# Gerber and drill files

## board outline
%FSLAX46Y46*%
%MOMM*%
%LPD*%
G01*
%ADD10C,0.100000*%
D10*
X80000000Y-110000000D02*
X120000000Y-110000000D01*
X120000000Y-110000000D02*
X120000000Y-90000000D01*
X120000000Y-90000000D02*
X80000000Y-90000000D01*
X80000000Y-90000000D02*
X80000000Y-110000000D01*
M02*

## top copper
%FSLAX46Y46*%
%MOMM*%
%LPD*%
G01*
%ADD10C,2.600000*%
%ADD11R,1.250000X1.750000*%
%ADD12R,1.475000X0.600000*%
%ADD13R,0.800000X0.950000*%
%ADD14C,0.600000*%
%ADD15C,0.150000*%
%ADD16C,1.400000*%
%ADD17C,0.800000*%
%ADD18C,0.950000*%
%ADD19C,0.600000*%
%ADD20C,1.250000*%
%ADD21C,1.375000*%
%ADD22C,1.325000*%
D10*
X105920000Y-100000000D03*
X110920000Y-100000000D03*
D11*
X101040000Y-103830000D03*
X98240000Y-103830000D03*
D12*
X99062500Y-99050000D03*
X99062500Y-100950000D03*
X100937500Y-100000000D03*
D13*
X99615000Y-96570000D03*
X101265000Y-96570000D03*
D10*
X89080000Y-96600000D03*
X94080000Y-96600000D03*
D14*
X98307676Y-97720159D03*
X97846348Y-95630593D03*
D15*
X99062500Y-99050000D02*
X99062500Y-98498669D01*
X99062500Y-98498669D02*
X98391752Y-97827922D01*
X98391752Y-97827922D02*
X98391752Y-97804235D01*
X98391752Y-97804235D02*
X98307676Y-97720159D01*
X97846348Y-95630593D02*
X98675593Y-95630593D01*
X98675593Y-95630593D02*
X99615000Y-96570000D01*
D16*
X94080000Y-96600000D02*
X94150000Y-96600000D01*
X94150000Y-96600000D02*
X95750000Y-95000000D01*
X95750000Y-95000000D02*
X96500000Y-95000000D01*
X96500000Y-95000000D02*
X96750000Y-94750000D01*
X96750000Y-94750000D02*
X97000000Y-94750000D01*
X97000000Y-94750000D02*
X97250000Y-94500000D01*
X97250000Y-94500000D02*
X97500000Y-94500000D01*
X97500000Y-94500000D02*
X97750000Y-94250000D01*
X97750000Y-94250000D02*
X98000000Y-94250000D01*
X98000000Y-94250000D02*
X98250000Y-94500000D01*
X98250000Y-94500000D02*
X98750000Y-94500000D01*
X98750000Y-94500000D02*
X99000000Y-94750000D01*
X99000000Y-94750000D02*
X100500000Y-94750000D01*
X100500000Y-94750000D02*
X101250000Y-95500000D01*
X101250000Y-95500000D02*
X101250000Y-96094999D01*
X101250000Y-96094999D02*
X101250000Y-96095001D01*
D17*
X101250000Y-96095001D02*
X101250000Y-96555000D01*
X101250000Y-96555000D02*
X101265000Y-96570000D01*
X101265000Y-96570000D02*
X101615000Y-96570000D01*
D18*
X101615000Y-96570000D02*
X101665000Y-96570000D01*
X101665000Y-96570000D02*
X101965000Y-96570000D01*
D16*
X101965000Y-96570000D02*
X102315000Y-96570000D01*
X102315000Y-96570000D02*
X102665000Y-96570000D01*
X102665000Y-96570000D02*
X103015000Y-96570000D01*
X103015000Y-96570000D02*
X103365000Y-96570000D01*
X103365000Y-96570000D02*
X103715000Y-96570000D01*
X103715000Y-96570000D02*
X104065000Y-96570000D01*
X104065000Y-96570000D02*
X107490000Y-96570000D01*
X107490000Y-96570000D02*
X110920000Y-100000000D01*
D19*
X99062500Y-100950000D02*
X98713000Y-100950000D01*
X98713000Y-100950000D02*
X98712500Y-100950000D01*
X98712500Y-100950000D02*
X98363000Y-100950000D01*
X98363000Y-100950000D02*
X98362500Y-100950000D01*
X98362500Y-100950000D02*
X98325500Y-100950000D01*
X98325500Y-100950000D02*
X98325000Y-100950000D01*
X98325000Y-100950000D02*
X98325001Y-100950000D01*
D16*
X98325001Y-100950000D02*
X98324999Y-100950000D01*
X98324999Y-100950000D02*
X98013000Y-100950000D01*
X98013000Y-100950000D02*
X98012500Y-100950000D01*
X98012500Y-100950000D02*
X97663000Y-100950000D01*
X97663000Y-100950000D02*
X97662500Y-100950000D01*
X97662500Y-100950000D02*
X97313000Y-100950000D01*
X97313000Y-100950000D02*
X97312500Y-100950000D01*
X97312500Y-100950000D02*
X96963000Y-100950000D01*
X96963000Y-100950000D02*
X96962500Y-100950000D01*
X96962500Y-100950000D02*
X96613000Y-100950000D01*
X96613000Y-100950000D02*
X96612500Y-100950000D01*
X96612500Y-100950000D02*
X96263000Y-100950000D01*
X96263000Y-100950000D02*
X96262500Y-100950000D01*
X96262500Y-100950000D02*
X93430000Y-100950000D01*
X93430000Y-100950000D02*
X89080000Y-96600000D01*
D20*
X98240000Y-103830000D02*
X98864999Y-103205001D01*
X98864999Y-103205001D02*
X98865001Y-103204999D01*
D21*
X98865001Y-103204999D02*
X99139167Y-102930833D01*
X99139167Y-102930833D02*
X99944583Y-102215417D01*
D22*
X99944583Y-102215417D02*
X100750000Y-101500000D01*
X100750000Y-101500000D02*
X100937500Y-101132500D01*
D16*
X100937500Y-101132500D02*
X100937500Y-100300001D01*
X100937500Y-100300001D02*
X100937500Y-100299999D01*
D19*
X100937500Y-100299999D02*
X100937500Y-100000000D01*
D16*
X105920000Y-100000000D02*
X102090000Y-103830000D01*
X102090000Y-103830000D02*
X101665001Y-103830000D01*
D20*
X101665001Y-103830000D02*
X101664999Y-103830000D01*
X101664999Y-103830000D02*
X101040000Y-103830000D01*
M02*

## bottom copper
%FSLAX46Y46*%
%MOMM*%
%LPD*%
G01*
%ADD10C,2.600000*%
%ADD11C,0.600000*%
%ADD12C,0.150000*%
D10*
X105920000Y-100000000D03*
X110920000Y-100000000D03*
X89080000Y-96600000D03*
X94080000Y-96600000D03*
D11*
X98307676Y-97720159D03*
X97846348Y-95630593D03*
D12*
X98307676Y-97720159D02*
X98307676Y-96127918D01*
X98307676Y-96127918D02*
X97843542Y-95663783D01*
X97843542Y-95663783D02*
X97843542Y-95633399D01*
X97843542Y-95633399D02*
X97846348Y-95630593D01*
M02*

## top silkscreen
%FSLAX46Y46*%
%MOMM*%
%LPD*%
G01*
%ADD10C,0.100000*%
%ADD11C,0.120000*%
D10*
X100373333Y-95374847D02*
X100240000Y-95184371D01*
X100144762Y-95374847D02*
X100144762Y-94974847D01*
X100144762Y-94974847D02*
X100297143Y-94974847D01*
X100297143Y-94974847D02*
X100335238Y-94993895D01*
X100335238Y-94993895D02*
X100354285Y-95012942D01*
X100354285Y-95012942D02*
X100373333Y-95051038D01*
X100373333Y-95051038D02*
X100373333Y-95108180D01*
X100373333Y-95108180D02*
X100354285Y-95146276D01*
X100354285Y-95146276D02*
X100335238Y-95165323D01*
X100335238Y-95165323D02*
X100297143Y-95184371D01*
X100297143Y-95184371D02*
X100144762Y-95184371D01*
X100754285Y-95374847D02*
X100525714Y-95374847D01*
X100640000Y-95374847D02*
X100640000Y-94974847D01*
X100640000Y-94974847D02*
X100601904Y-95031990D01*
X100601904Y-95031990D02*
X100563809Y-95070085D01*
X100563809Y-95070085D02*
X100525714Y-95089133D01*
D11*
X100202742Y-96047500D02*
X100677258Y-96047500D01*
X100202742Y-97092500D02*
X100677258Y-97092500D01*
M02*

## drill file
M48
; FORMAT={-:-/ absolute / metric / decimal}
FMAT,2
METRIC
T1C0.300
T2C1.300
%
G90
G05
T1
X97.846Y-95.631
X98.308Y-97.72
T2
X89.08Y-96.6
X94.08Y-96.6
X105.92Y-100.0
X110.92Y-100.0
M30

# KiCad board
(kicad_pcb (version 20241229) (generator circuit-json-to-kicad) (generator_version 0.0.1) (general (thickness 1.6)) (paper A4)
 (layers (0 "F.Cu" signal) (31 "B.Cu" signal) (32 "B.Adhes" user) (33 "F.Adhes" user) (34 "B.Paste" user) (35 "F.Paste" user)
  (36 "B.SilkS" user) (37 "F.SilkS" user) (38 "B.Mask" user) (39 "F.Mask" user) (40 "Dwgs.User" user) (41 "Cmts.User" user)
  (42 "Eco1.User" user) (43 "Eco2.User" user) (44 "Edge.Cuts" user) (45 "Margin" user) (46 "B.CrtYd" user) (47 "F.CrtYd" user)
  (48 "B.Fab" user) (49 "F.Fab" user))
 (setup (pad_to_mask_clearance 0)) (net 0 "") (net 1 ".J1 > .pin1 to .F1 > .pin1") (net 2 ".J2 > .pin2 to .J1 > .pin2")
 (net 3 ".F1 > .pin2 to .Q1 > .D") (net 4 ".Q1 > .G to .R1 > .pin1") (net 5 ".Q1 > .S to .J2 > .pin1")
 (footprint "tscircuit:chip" (layer F.Cu) (at 105.92 100 0)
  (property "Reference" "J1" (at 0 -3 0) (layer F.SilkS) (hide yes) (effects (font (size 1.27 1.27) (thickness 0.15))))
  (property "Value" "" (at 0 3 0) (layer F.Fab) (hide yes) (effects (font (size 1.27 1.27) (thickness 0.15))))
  (pad "1" thru_hole circle (at 0 0 0) (size 2.6 2.6) (drill 1.3) (layers *.Cu *.Mask) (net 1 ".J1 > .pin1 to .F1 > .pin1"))
  (pad "2" thru_hole circle (at 5 0 0) (size 2.6 2.6) (drill 1.3) (layers *.Cu *.Mask) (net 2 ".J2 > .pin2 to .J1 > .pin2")))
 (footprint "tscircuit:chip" (layer F.Cu) (at 99.64 103.83 180)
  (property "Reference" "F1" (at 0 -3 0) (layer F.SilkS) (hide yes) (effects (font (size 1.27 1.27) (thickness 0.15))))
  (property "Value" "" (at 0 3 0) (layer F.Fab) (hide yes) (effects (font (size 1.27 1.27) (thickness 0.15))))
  (pad "1" smd rect (at -1.4 0 0) (size 1.25 1.75) (layers F.Cu F.Mask) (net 1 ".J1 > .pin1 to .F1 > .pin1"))
  (pad "2" smd rect (at 1.4 0 0) (size 1.25 1.75) (layers F.Cu F.Mask) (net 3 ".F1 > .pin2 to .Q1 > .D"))
  (pad "" smd rect (at -1.4 0 0) (size 0.875 1.2249999999999999) (layers F.Paste))
  (pad "" smd rect (at 1.4 0 0) (size 0.875 1.2249999999999999) (layers F.Paste)))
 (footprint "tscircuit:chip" (layer F.Cu) (at 100 100 0)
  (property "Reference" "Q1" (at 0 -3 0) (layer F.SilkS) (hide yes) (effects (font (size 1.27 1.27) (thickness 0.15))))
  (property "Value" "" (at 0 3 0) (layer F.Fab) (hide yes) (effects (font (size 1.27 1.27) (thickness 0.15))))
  (pad "1" smd rect (at -0.9375 -0.95 0) (size 1.475 0.6) (layers F.Cu F.Mask) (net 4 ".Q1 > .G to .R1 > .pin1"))
  (pad "2" smd rect (at -0.9375 0.95 0) (size 1.475 0.6) (layers F.Cu F.Mask) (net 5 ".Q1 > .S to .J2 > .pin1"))
  (pad "3" smd rect (at 0.9375 0 0) (size 1.475 0.6) (layers F.Cu F.Mask) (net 3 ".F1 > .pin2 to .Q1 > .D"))
  (pad "" smd rect (at -0.9375 -0.95 0) (size 1.0325 0.42) (layers F.Paste))
  (pad "" smd rect (at -0.9375 0.95 0) (size 1.0325 0.42) (layers F.Paste))
  (pad "" smd rect (at 0.9375 0 0) (size 1.0325 0.42) (layers F.Paste)))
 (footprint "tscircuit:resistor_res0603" (layer F.Cu) (at 100.44 96.57 0)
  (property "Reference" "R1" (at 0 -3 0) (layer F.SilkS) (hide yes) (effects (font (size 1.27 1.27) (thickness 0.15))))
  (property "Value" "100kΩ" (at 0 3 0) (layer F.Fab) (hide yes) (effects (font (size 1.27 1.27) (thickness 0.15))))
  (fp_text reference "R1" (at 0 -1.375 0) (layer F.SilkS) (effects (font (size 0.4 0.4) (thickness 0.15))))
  (fp_line (start -0.237258 -0.5225) (end 0.23725799999999997 -0.5225) (stroke (width 0.12) (type default)) (layer F.SilkS))
  (fp_line (start -0.237258 0.5225) (end 0.23725799999999997 0.5225) (stroke (width 0.12) (type default)) (layer F.SilkS))
  (pad "1" smd rect (at -0.825 0 0) (size 0.8 0.95) (layers F.Cu F.Mask) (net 4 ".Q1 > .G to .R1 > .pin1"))
  (pad "2" smd rect (at 0.825 0 0) (size 0.8 0.95) (layers F.Cu F.Mask) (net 2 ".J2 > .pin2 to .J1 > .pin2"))
  (pad "" smd rect (at -0.825 0 0) (size 0.5599999999999999 0.6649999999999999) (layers F.Paste))
  (pad "" smd rect (at 0.825 0 0) (size 0.5599999999999999 0.6649999999999999) (layers F.Paste)))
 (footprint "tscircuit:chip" (layer F.Cu) (at 89.08 96.6 0)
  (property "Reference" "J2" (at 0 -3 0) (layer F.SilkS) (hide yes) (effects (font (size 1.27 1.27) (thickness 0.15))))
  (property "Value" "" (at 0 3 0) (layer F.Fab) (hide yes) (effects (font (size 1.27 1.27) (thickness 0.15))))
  (pad "1" thru_hole circle (at 0 0 0) (size 2.6 2.6) (drill 1.3) (layers *.Cu *.Mask) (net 5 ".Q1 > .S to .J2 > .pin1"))
  (pad "2" thru_hole circle (at 5 0 0) (size 2.6 2.6) (drill 1.3) (layers *.Cu *.Mask) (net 2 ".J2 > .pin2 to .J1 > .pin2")))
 (segment (start 99.0625 99.05) (end 99.0625 98.49866917639389) (width 0.15) (layer F.Cu) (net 4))
 (segment (start 99.0625 98.49866917639389) (end 98.39175243083571 97.82792160722961) (width 0.15) (layer F.Cu) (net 4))
 (segment (start 98.39175243083571 97.82792160722961) (end 98.39175243083571 97.80423524011546) (width 0.15) (layer F.Cu) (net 4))
 (segment (start 98.39175243083571 97.80423524011546) (end 98.30767637246909 97.72015918174884) (width 0.15) (layer F.Cu) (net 4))
 (segment (start 98.30767637246909 97.72015918174884) (end 98.30767637246909 96.12791807272515) (width 0.15) (layer B.Cu) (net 4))
 (segment (start 98.30767637246909 96.12791807272515) (end 97.84354177922641 95.66378347948246) (width 0.15) (layer B.Cu) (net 4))
 (segment (start 97.84354177922641 95.66378347948246) (end 97.84354177922641 95.63339917294248) (width 0.15) (layer B.Cu) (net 4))
 (segment (start 97.84354177922641 95.63339917294248) (end 97.8463483227921 95.63059262937678) (width 0.15) (layer B.Cu) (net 4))
 (segment (start 97.8463483227921 95.63059262937678) (end 98.67559262937678 95.63059262937678) (width 0.15) (layer F.Cu) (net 4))
 (segment (start 98.67559262937678 95.63059262937678) (end 99.615 96.57) (width 0.15) (layer F.Cu) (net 4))
 (segment (start 94.08 96.6) (end 94.15 96.6) (width 1.4) (layer F.Cu) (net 2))
 (segment (start 94.15 96.6) (end 95.75 95) (width 1.4) (layer F.Cu) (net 2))
 (segment (start 95.75 95) (end 96.5 95) (width 1.4) (layer F.Cu) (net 2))
 (segment (start 96.5 95) (end 96.75 94.75) (width 1.4) (layer F.Cu) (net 2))
 (segment (start 96.75 94.75) (end 97 94.75) (width 1.4) (layer F.Cu) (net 2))
 (segment (start 97 94.75) (end 97.25 94.5) (width 1.4) (layer F.Cu) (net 2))
 (segment (start 97.25 94.5) (end 97.5 94.5) (width 1.4) (layer F.Cu) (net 2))
 (segment (start 97.5 94.5) (end 97.75 94.25) (width 1.4) (layer F.Cu) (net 2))
 (segment (start 97.75 94.25) (end 98 94.25) (width 1.4) (layer F.Cu) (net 2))
 (segment (start 98 94.25) (end 98.25 94.5) (width 1.4) (layer F.Cu) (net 2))
 (segment (start 98.25 94.5) (end 98.75 94.5) (width 1.4) (layer F.Cu) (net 2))
 (segment (start 98.75 94.5) (end 99 94.75) (width 1.4) (layer F.Cu) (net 2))
 (segment (start 99 94.75) (end 100.5 94.75) (width 1.4) (layer F.Cu) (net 2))
 (segment (start 100.5 94.75) (end 101.25 95.5) (width 1.4) (layer F.Cu) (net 2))
 (segment (start 101.25 95.5) (end 101.25 96.094999) (width 1.4) (layer F.Cu) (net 2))
 (segment (start 101.25 96.094999) (end 101.25 96.095001) (width 1.4) (layer F.Cu) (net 2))
 (segment (start 101.25 96.095001) (end 101.25 96.555) (width 0.8) (layer F.Cu) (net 2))
 (segment (start 101.25 96.555) (end 101.265 96.57) (width 0.8) (layer F.Cu) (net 2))
 (segment (start 101.265 96.57) (end 101.615 96.57) (width 0.8) (layer F.Cu) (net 2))
 (segment (start 101.615 96.57) (end 101.665 96.57) (width 0.95) (layer F.Cu) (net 2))
 (segment (start 101.665 96.57) (end 101.965 96.57) (width 0.95) (layer F.Cu) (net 2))
 (segment (start 101.965 96.57) (end 102.315 96.57) (width 1.4) (layer F.Cu) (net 2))
 (segment (start 102.315 96.57) (end 102.665 96.57) (width 1.4) (layer F.Cu) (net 2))
 (segment (start 102.665 96.57) (end 103.015 96.57) (width 1.4) (layer F.Cu) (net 2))
 (segment (start 103.015 96.57) (end 103.365 96.57) (width 1.4) (layer F.Cu) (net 2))
 (segment (start 103.365 96.57) (end 103.715 96.57) (width 1.4) (layer F.Cu) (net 2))
 (segment (start 103.715 96.57) (end 104.065 96.57) (width 1.4) (layer F.Cu) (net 2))
 (segment (start 104.065 96.57) (end 107.49 96.57) (width 1.4) (layer F.Cu) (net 2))
 (segment (start 107.49 96.57) (end 110.92 100) (width 1.4) (layer F.Cu) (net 2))
 (segment (start 99.0625 100.95) (end 98.713 100.95) (width 0.6) (layer F.Cu) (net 5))
 (segment (start 98.713 100.95) (end 98.7125 100.95) (width 0.6) (layer F.Cu) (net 5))
 (segment (start 98.7125 100.95) (end 98.363 100.95) (width 0.6) (layer F.Cu) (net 5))
 (segment (start 98.363 100.95) (end 98.3625 100.95) (width 0.6) (layer F.Cu) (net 5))
 (segment (start 98.3625 100.95) (end 98.3255 100.95) (width 0.6) (layer F.Cu) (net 5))
 (segment (start 98.3255 100.95) (end 98.325 100.95) (width 0.6) (layer F.Cu) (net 5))
 (segment (start 98.325 100.95) (end 98.325001 100.95) (width 0.6) (layer F.Cu) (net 5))
 (segment (start 98.325001 100.95) (end 98.324999 100.95) (width 1.4) (layer F.Cu) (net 5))
 (segment (start 98.324999 100.95) (end 98.013 100.95) (width 1.4) (layer F.Cu) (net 5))
 (segment (start 98.013 100.95) (end 98.0125 100.95) (width 1.4) (layer F.Cu) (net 5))
 (segment (start 98.0125 100.95) (end 97.663 100.95) (width 1.4) (layer F.Cu) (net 5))
 (segment (start 97.663 100.95) (end 97.6625 100.95) (width 1.4) (layer F.Cu) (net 5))
 (segment (start 97.6625 100.95) (end 97.313 100.95) (width 1.4) (layer F.Cu) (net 5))
 (segment (start 97.313 100.95) (end 97.3125 100.95) (width 1.4) (layer F.Cu) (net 5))
 (segment (start 97.3125 100.95) (end 96.963 100.95) (width 1.4) (layer F.Cu) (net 5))
 (segment (start 96.963 100.95) (end 96.9625 100.95) (width 1.4) (layer F.Cu) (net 5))
 (segment (start 96.9625 100.95) (end 96.613 100.95) (width 1.4) (layer F.Cu) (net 5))
 (segment (start 96.613 100.95) (end 96.6125 100.95) (width 1.4) (layer F.Cu) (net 5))
 (segment (start 96.6125 100.95) (end 96.263 100.95) (width 1.4) (layer F.Cu) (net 5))
 (segment (start 96.263 100.95) (end 96.2625 100.95) (width 1.4) (layer F.Cu) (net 5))
 (segment (start 96.2625 100.95) (end 93.42999999999999 100.95) (width 1.4) (layer F.Cu) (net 5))
 (segment (start 93.42999999999999 100.95) (end 89.08 96.6) (width 1.4) (layer F.Cu) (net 5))
 (segment (start 98.24 103.83) (end 98.86499929289322 103.20500070710678) (width 1.25) (layer F.Cu) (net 3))
 (segment (start 98.86499929289322 103.20500070710678) (end 98.86500070710679 103.20499929289322) (width 1.25) (layer F.Cu) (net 3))
 (segment (start 98.86500070710679 103.20499929289322) (end 99.13916666666667 102.93083333333334) (width 1.375) (layer F.Cu) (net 3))
 (segment (start 99.13916666666667 102.93083333333334) (end 99.94458333333333 102.21541666666667) (width 1.375) (layer F.Cu) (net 3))
 (segment (start 99.94458333333333 102.21541666666667) (end 100.75 101.5) (width 1.3250000000000002) (layer F.Cu) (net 3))
 (segment (start 100.75 101.5) (end 100.9375 101.1325) (width 1.3250000000000002) (layer F.Cu) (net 3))
 (segment (start 100.9375 101.1325) (end 100.9375 100.300001) (width 1.4) (layer F.Cu) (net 3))
 (segment (start 100.9375 100.300001) (end 100.9375 100.299999) (width 1.4) (layer F.Cu) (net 3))
 (segment (start 100.9375 100.299999) (end 100.9375 100) (width 0.6) (layer F.Cu) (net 3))
 (segment (start 105.92 100) (end 102.09 103.83) (width 1.4) (layer F.Cu) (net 1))
 (segment (start 102.09 103.83) (end 101.665001 103.83) (width 1.4) (layer F.Cu) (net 1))
 (segment (start 101.665001 103.83) (end 101.664999 103.83) (width 1.25) (layer F.Cu) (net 1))
 (segment (start 101.664999 103.83) (end 101.04 103.83) (width 1.25) (layer F.Cu) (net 1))
 (gr_line (start 80 110) (end 120 110) (width 0.1) (layer Edge.Cuts))
 (gr_line (start 120 110) (end 120 90) (width 0.1) (layer Edge.Cuts))
 (gr_line (start 120 90) (end 80 90) (width 0.1) (layer Edge.Cuts))
 (gr_line (start 80 90) (end 80 110) (width 0.1) (layer Edge.Cuts))
 (via (at 98.30767637246909 97.72015918174884) (size 0.6) (drill 0.3) (layers F.Cu B.Cu) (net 4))
 (via (at 97.8463483227921 95.63059262937678) (size 0.6) (drill 0.3) (layers F.Cu B.Cu) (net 4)))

